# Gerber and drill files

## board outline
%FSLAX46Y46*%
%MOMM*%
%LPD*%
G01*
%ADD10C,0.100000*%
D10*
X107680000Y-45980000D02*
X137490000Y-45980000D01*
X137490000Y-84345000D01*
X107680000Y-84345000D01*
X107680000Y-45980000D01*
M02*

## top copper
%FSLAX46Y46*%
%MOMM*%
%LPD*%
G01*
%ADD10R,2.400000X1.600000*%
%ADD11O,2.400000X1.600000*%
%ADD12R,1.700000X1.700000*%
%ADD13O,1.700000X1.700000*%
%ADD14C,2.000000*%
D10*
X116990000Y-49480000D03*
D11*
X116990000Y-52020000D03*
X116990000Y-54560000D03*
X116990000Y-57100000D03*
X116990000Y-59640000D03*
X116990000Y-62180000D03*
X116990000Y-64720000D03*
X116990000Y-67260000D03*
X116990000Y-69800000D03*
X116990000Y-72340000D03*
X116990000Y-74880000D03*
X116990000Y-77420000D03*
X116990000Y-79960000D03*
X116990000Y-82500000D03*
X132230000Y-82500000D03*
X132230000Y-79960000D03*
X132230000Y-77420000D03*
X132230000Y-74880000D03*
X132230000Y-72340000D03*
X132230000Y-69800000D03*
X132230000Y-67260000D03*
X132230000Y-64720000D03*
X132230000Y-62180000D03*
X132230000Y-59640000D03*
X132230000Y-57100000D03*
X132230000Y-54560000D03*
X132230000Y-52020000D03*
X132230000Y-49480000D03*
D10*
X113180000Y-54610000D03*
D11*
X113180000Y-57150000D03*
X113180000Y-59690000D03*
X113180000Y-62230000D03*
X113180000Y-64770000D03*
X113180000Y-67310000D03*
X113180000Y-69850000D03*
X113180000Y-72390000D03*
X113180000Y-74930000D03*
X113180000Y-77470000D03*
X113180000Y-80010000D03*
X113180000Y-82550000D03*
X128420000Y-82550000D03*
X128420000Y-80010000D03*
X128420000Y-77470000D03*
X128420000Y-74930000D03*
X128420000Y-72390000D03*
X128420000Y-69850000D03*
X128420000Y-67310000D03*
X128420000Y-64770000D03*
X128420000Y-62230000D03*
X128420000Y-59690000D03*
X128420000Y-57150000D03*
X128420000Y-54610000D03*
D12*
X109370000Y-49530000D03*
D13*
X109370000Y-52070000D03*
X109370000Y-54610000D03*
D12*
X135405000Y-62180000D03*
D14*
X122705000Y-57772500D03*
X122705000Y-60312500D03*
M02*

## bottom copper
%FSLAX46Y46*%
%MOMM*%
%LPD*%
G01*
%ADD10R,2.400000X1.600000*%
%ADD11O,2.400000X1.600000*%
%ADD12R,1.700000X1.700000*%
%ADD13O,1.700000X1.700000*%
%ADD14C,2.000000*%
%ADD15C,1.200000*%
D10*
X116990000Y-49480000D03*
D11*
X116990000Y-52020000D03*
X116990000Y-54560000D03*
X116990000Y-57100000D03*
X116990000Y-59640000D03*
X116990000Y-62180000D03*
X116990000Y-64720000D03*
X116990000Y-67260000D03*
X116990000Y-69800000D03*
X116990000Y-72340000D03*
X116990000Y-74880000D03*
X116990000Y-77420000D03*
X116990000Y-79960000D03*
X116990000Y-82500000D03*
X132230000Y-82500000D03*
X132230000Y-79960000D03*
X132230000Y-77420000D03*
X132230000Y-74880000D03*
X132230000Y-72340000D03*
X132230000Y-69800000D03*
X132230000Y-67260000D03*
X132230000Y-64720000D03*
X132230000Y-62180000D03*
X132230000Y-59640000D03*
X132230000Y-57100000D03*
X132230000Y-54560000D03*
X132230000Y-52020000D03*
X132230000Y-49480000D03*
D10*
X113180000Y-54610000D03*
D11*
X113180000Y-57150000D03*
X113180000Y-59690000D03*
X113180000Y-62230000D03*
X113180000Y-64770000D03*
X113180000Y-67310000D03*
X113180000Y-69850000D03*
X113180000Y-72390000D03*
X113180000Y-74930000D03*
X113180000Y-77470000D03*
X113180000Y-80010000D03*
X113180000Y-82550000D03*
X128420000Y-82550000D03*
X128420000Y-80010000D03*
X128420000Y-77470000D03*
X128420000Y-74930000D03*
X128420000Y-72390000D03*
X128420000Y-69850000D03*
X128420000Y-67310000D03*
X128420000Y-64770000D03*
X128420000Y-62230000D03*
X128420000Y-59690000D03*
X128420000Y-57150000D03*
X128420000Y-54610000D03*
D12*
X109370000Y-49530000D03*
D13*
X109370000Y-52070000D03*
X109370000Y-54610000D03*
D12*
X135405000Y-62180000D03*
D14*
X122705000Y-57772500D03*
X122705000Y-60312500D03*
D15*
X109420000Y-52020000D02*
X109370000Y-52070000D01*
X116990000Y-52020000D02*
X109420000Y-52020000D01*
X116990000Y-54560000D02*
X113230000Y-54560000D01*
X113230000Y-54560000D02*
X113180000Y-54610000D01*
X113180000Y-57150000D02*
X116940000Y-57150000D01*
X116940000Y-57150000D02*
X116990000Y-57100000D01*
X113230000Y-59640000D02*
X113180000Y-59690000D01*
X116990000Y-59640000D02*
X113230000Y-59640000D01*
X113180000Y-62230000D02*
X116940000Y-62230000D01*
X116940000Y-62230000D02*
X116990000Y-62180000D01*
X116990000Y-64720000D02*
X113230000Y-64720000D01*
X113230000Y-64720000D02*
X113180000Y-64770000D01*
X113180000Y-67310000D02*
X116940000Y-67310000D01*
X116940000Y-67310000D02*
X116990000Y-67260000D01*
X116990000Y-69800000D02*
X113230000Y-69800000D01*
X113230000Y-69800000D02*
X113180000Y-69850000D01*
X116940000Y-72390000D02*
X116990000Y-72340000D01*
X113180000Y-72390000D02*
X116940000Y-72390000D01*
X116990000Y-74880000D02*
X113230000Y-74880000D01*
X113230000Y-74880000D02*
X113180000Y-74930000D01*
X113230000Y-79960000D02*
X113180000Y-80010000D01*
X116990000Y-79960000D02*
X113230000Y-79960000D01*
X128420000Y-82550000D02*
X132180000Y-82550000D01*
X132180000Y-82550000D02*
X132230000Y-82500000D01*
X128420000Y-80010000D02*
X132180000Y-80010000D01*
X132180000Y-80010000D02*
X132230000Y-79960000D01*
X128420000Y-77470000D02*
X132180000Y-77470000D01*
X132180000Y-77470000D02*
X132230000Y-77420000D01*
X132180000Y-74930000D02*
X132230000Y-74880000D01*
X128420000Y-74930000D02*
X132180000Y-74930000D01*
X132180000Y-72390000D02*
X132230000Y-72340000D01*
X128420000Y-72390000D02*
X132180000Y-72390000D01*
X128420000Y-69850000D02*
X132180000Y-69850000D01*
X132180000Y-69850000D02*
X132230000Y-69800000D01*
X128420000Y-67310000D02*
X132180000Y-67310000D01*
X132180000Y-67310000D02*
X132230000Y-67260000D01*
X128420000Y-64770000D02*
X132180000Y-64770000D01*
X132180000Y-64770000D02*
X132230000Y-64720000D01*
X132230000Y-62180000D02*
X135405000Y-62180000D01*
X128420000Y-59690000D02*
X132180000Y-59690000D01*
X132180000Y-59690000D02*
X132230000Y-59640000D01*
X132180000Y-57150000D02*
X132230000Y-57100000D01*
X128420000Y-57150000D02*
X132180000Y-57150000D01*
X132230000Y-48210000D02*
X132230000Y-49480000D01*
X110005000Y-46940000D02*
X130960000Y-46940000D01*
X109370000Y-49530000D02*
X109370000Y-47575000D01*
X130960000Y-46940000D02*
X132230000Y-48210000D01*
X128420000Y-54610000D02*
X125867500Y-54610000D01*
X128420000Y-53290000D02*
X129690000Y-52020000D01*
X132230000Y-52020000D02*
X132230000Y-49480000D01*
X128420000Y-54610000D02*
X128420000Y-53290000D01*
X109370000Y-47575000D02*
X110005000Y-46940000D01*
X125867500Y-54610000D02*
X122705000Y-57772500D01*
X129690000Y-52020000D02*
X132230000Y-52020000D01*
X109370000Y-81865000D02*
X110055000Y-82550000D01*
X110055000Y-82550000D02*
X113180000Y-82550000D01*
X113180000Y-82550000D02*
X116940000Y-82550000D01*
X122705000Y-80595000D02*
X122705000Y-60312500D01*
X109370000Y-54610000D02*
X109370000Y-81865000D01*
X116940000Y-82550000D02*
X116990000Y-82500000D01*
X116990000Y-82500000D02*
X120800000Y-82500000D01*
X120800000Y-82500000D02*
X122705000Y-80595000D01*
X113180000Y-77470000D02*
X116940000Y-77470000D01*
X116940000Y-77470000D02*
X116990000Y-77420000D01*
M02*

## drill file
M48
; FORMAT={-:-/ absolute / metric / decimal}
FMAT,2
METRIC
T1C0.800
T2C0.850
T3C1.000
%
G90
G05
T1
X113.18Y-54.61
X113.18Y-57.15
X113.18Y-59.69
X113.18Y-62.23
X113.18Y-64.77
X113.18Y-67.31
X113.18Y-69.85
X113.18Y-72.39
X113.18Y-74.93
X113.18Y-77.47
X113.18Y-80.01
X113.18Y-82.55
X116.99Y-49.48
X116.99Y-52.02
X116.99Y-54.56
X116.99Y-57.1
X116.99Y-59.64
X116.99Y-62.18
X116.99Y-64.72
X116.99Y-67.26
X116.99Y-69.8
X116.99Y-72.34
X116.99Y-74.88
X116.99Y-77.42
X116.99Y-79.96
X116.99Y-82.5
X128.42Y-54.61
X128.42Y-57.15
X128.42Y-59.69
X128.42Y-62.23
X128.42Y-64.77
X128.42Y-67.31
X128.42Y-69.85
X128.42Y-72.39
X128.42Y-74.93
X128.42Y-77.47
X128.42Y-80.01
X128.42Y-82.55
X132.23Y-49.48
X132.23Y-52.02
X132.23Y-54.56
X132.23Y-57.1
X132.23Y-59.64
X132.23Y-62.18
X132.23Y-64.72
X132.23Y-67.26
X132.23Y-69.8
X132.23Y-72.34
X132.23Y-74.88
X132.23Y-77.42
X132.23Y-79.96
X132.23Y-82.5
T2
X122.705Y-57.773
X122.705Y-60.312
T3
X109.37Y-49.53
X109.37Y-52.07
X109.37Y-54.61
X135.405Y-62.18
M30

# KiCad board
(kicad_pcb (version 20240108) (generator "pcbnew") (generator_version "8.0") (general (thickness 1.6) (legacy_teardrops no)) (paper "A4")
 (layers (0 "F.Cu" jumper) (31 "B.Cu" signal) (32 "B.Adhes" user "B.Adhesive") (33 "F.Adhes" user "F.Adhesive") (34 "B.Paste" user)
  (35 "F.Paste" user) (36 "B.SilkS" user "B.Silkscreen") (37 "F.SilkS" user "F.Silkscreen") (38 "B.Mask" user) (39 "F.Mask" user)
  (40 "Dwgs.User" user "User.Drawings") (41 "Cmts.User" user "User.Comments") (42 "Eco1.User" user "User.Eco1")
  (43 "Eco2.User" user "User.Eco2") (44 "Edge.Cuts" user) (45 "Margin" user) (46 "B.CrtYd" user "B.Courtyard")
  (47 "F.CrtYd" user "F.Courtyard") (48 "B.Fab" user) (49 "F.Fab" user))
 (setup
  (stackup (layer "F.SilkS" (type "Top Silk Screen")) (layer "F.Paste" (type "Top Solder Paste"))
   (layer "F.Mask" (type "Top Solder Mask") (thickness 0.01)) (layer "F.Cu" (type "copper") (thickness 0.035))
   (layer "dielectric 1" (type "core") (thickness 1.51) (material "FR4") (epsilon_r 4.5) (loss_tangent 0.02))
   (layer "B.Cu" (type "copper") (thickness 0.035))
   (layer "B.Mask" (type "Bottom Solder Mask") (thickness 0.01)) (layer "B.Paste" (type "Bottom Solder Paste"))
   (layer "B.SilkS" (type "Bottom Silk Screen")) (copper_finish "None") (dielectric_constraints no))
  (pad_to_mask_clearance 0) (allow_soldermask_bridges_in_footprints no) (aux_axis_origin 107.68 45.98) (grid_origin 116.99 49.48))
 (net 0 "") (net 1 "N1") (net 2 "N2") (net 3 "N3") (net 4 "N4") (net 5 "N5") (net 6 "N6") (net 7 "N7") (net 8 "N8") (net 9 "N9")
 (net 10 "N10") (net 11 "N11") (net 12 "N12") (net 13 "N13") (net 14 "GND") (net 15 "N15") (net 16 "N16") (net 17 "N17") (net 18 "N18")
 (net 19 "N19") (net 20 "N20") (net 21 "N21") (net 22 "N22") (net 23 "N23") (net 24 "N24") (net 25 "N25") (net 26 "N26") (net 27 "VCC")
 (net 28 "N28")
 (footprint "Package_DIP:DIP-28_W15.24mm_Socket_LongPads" (layer "F.Cu") (at 116.99 49.48)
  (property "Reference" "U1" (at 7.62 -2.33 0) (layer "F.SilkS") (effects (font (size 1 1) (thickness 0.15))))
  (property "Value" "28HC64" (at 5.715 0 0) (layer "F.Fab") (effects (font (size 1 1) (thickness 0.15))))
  (pad "1" thru_hole rect (at 0 0) (size 2.4 1.6) (drill 0.8) (layers "*.Cu" "*.Mask") (remove_unused_layers no) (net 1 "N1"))
  (pad "2" thru_hole oval (at 0 2.54) (size 2.4 1.6) (drill 0.8) (layers "*.Cu" "*.Mask") (remove_unused_layers no) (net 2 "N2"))
  (pad "3" thru_hole oval (at 0 5.08) (size 2.4 1.6) (drill 0.8) (layers "*.Cu" "*.Mask") (remove_unused_layers no) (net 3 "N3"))
  (pad "4" thru_hole oval (at 0 7.62) (size 2.4 1.6) (drill 0.8) (layers "*.Cu" "*.Mask") (remove_unused_layers no) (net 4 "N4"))
  (pad "5" thru_hole oval (at 0 10.16) (size 2.4 1.6) (drill 0.8) (layers "*.Cu" "*.Mask") (remove_unused_layers no) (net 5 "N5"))
  (pad "6" thru_hole oval (at 0 12.7) (size 2.4 1.6) (drill 0.8) (layers "*.Cu" "*.Mask") (remove_unused_layers no) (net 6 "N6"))
  (pad "7" thru_hole oval (at 0 15.24) (size 2.4 1.6) (drill 0.8) (layers "*.Cu" "*.Mask") (remove_unused_layers no) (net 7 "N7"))
  (pad "8" thru_hole oval (at 0 17.78) (size 2.4 1.6) (drill 0.8) (layers "*.Cu" "*.Mask") (remove_unused_layers no) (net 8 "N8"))
  (pad "9" thru_hole oval (at 0 20.32) (size 2.4 1.6) (drill 0.8) (layers "*.Cu" "*.Mask") (remove_unused_layers no) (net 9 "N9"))
  (pad "10" thru_hole oval (at 0 22.86) (size 2.4 1.6) (drill 0.8) (layers "*.Cu" "*.Mask") (remove_unused_layers no) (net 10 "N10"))
  (pad "11" thru_hole oval (at 0 25.4) (size 2.4 1.6) (drill 0.8) (layers "*.Cu" "*.Mask") (remove_unused_layers no) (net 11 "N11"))
  (pad "12" thru_hole oval (at 0 27.94) (size 2.4 1.6) (drill 0.8) (layers "*.Cu" "*.Mask") (remove_unused_layers no) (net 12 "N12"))
  (pad "13" thru_hole oval (at 0 30.48) (size 2.4 1.6) (drill 0.8) (layers "*.Cu" "*.Mask") (remove_unused_layers no) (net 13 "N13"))
  (pad "14" thru_hole oval (at 0 33.02) (size 2.4 1.6) (drill 0.8) (layers "*.Cu" "*.Mask") (remove_unused_layers no) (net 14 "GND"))
  (pad "15" thru_hole oval (at 15.24 33.02) (size 2.4 1.6) (drill 0.8) (layers "*.Cu" "*.Mask") (remove_unused_layers no) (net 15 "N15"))
  (pad "16" thru_hole oval (at 15.24 30.48) (size 2.4 1.6) (drill 0.8) (layers "*.Cu" "*.Mask") (remove_unused_layers no) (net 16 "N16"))
  (pad "17" thru_hole oval (at 15.24 27.94) (size 2.4 1.6) (drill 0.8) (layers "*.Cu" "*.Mask") (remove_unused_layers no) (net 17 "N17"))
  (pad "18" thru_hole oval (at 15.24 25.4) (size 2.4 1.6) (drill 0.8) (layers "*.Cu" "*.Mask") (remove_unused_layers no) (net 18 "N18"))
  (pad "19" thru_hole oval (at 15.24 22.86) (size 2.4 1.6) (drill 0.8) (layers "*.Cu" "*.Mask") (remove_unused_layers no) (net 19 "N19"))
  (pad "20" thru_hole oval (at 15.24 20.32) (size 2.4 1.6) (drill 0.8) (layers "*.Cu" "*.Mask") (remove_unused_layers no) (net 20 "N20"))
  (pad "21" thru_hole oval (at 15.24 17.78) (size 2.4 1.6) (drill 0.8) (layers "*.Cu" "*.Mask") (remove_unused_layers no) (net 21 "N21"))
  (pad "22" thru_hole oval (at 15.24 15.24) (size 2.4 1.6) (drill 0.8) (layers "*.Cu" "*.Mask") (remove_unused_layers no) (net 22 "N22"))
  (pad "23" thru_hole oval (at 15.24 12.7) (size 2.4 1.6) (drill 0.8) (layers "*.Cu" "*.Mask") (remove_unused_layers no) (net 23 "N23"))
  (pad "24" thru_hole oval (at 15.24 10.16) (size 2.4 1.6) (drill 0.8) (layers "*.Cu" "*.Mask") (remove_unused_layers no) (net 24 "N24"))
  (pad "25" thru_hole oval (at 15.24 7.62) (size 2.4 1.6) (drill 0.8) (layers "*.Cu" "*.Mask") (remove_unused_layers no) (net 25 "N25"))
  (pad "26" thru_hole oval (at 15.24 5.08) (size 2.4 1.6) (drill 0.8) (layers "*.Cu" "*.Mask") (remove_unused_layers no) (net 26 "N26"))
  (pad "27" thru_hole oval (at 15.24 2.54) (size 2.4 1.6) (drill 0.8) (layers "*.Cu" "*.Mask") (remove_unused_layers no) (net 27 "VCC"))
  (pad "28" thru_hole oval (at 15.24 0) (size 2.4 1.6) (drill 0.8) (layers "*.Cu" "*.Mask") (remove_unused_layers no) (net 27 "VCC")))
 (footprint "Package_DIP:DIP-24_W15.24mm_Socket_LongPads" (layer "F.Cu") (at 113.18 54.61)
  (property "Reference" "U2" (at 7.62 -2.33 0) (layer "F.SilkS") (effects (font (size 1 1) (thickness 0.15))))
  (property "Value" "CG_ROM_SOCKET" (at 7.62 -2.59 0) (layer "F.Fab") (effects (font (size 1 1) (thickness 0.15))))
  (pad "1" thru_hole rect (at 0 0) (size 2.4 1.6) (drill 0.8) (layers "*.Cu" "*.Mask") (remove_unused_layers no) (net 3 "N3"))
  (pad "2" thru_hole oval (at 0 2.54) (size 2.4 1.6) (drill 0.8) (layers "*.Cu" "*.Mask") (remove_unused_layers no) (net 4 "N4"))
  (pad "3" thru_hole oval (at 0 5.08) (size 2.4 1.6) (drill 0.8) (layers "*.Cu" "*.Mask") (remove_unused_layers no) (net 5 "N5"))
  (pad "4" thru_hole oval (at 0 7.62) (size 2.4 1.6) (drill 0.8) (layers "*.Cu" "*.Mask") (remove_unused_layers no) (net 6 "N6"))
  (pad "5" thru_hole oval (at 0 10.16) (size 2.4 1.6) (drill 0.8) (layers "*.Cu" "*.Mask") (remove_unused_layers no) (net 7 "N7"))
  (pad "6" thru_hole oval (at 0 12.7) (size 2.4 1.6) (drill 0.8) (layers "*.Cu" "*.Mask") (remove_unused_layers no) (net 8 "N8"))
  (pad "7" thru_hole oval (at 0 15.24) (size 2.4 1.6) (drill 0.8) (layers "*.Cu" "*.Mask") (remove_unused_layers no) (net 9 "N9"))
  (pad "8" thru_hole oval (at 0 17.78) (size 2.4 1.6) (drill 0.8) (layers "*.Cu" "*.Mask") (remove_unused_layers no) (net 10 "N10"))
  (pad "9" thru_hole oval (at 0 20.32) (size 2.4 1.6) (drill 0.8) (layers "*.Cu" "*.Mask") (remove_unused_layers no) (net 11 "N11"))
  (pad "10" thru_hole oval (at 0 22.86) (size 2.4 1.6) (drill 0.8) (layers "*.Cu" "*.Mask") (remove_unused_layers no) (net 12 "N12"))
  (pad "11" thru_hole oval (at 0 25.4) (size 2.4 1.6) (drill 0.8) (layers "*.Cu" "*.Mask") (remove_unused_layers no) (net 13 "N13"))
  (pad "12" thru_hole oval (at 0 27.94) (size 2.4 1.6) (drill 0.8) (layers "*.Cu" "*.Mask") (remove_unused_layers no) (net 14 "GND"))
  (pad "13" thru_hole oval (at 15.24 27.94) (size 2.4 1.6) (drill 0.8) (layers "*.Cu" "*.Mask") (remove_unused_layers no) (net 15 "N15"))
  (pad "14" thru_hole oval (at 15.24 25.4) (size 2.4 1.6) (drill 0.8) (layers "*.Cu" "*.Mask") (remove_unused_layers no) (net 16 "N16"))
  (pad "15" thru_hole oval (at 15.24 22.86) (size 2.4 1.6) (drill 0.8) (layers "*.Cu" "*.Mask") (remove_unused_layers no) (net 17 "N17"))
  (pad "16" thru_hole oval (at 15.24 20.32) (size 2.4 1.6) (drill 0.8) (layers "*.Cu" "*.Mask") (remove_unused_layers no) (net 18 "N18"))
  (pad "17" thru_hole oval (at 15.24 17.78) (size 2.4 1.6) (drill 0.8) (layers "*.Cu" "*.Mask") (remove_unused_layers no) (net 19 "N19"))
  (pad "18" thru_hole oval (at 15.24 15.24) (size 2.4 1.6) (drill 0.8) (layers "*.Cu" "*.Mask") (remove_unused_layers no) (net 20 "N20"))
  (pad "19" thru_hole oval (at 15.24 12.7) (size 2.4 1.6) (drill 0.8) (layers "*.Cu" "*.Mask") (remove_unused_layers no) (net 21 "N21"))
  (pad "20" thru_hole oval (at 15.24 10.16) (size 2.4 1.6) (drill 0.8) (layers "*.Cu" "*.Mask") (remove_unused_layers no) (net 22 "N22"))
  (pad "21" thru_hole oval (at 15.24 7.62) (size 2.4 1.6) (drill 0.8) (layers "*.Cu" "*.Mask") (remove_unused_layers no) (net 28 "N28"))
  (pad "22" thru_hole oval (at 15.24 5.08) (size 2.4 1.6) (drill 0.8) (layers "*.Cu" "*.Mask") (remove_unused_layers no) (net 24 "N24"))
  (pad "23" thru_hole oval (at 15.24 2.54) (size 2.4 1.6) (drill 0.8) (layers "*.Cu" "*.Mask") (remove_unused_layers no) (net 25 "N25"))
  (pad "24" thru_hole oval (at 15.24 0) (size 2.4 1.6) (drill 0.8) (layers "*.Cu" "*.Mask") (remove_unused_layers no) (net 27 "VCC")))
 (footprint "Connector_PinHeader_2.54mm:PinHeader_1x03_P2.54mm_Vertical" (layer "F.Cu") (at 109.37 49.53)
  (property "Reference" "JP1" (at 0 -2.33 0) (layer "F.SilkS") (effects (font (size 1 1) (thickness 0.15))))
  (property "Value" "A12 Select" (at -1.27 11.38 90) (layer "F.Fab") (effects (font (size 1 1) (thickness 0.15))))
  (pad "1" thru_hole rect (at 0 0) (size 1.7 1.7) (drill 1) (layers "*.Cu" "*.Mask") (remove_unused_layers no) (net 27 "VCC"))
  (pad "2" thru_hole oval (at 0 2.54) (size 1.7 1.7) (drill 1) (layers "*.Cu" "*.Mask") (remove_unused_layers no) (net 2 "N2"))
  (pad "3" thru_hole oval (at 0 5.08) (size 1.7 1.7) (drill 1) (layers "*.Cu" "*.Mask") (remove_unused_layers no) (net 14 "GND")))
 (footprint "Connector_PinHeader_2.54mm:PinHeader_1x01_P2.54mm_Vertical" (layer "F.Cu") (at 135.405 62.18)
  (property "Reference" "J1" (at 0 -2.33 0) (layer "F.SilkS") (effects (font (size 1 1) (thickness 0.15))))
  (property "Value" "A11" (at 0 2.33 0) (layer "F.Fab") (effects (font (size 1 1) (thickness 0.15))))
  (pad "1" thru_hole rect (at 0 0) (size 1.7 1.7) (drill 1) (layers "*.Cu" "*.Mask") (remove_unused_layers no) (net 23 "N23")))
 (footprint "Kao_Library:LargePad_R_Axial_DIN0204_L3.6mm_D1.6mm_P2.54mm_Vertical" (layer "F.Cu") (at 122.705 57.7725 -90)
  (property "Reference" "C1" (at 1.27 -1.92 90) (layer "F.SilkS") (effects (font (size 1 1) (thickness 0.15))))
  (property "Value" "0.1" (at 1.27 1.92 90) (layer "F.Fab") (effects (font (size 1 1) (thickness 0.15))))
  (pad "1" thru_hole circle (at 0 0 270) (size 2 2) (drill 0.85) (layers "*.Cu" "*.Mask") (remove_unused_layers no) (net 27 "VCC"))
  (pad "2" thru_hole circle (at 2.54 0 270) (size 2 2) (drill 0.85) (layers "*.Cu" "*.Mask") (remove_unused_layers no) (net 14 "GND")))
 (gr_rect (start 107.68 45.98) (end 137.49 84.345) (stroke (width 0.1) (type default)) (fill none) (layer "Edge.Cuts"))
 (segment (start 109.42 52.02) (end 109.37 52.07) (width 1.2) (layer "B.Cu") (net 2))
 (segment (start 116.99 52.02) (end 109.42 52.02) (width 1.2) (layer "B.Cu") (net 2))
 (segment (start 116.99 54.56) (end 113.23 54.56) (width 1.2) (layer "B.Cu") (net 3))
 (segment (start 113.23 54.56) (end 113.18 54.61) (width 1.2) (layer "B.Cu") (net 3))
 (segment (start 113.18 57.15) (end 116.94 57.15) (width 1.2) (layer "B.Cu") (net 4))
 (segment (start 116.94 57.15) (end 116.99 57.1) (width 1.2) (layer "B.Cu") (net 4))
 (segment (start 113.23 59.64) (end 113.18 59.69) (width 1.2) (layer "B.Cu") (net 5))
 (segment (start 116.99 59.64) (end 113.23 59.64) (width 1.2) (layer "B.Cu") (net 5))
 (segment (start 113.18 62.23) (end 116.94 62.23) (width 1.2) (layer "B.Cu") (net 6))
 (segment (start 116.94 62.23) (end 116.99 62.18) (width 1.2) (layer "B.Cu") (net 6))
 (segment (start 116.99 64.72) (end 113.23 64.72) (width 1.2) (layer "B.Cu") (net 7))
 (segment (start 113.23 64.72) (end 113.18 64.77) (width 1.2) (layer "B.Cu") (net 7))
 (segment (start 113.18 67.31) (end 116.94 67.31) (width 1.2) (layer "B.Cu") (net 8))
 (segment (start 116.94 67.31) (end 116.99 67.26) (width 1.2) (layer "B.Cu") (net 8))
 (segment (start 116.99 69.8) (end 113.23 69.8) (width 1.2) (layer "B.Cu") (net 9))
 (segment (start 113.23 69.8) (end 113.18 69.85) (width 1.2) (layer "B.Cu") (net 9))
 (segment (start 116.94 72.39) (end 116.99 72.34) (width 1.2) (layer "B.Cu") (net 10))
 (segment (start 113.18 72.39) (end 116.94 72.39) (width 1.2) (layer "B.Cu") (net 10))
 (segment (start 116.99 74.88) (end 113.23 74.88) (width 1.2) (layer "B.Cu") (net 11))
 (segment (start 113.23 74.88) (end 113.18 74.93) (width 1.2) (layer "B.Cu") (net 11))
 (segment (start 113.23 79.96) (end 113.18 80.01) (width 1.2) (layer "B.Cu") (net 13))
 (segment (start 116.99 79.96) (end 113.23 79.96) (width 1.2) (layer "B.Cu") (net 13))
 (segment (start 128.42 82.55) (end 132.18 82.55) (width 1.2) (layer "B.Cu") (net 15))
 (segment (start 132.18 82.55) (end 132.23 82.5) (width 1.2) (layer "B.Cu") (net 15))
 (segment (start 128.42 80.01) (end 132.18 80.01) (width 1.2) (layer "B.Cu") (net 16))
 (segment (start 132.18 80.01) (end 132.23 79.96) (width 1.2) (layer "B.Cu") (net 16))
 (segment (start 128.42 77.47) (end 132.18 77.47) (width 1.2) (layer "B.Cu") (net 17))
 (segment (start 132.18 77.47) (end 132.23 77.42) (width 1.2) (layer "B.Cu") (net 17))
 (segment (start 132.18 74.93) (end 132.23 74.88) (width 1.2) (layer "B.Cu") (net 18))
 (segment (start 128.42 74.93) (end 132.18 74.93) (width 1.2) (layer "B.Cu") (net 18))
 (segment (start 132.18 72.39) (end 132.23 72.34) (width 1.2) (layer "B.Cu") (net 19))
 (segment (start 128.42 72.39) (end 132.18 72.39) (width 1.2) (layer "B.Cu") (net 19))
 (segment (start 128.42 69.85) (end 132.18 69.85) (width 1.2) (layer "B.Cu") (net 20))
 (segment (start 132.18 69.85) (end 132.23 69.8) (width 1.2) (layer "B.Cu") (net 20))
 (segment (start 128.42 67.31) (end 132.18 67.31) (width 1.2) (layer "B.Cu") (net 21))
 (segment (start 132.18 67.31) (end 132.23 67.26) (width 1.2) (layer "B.Cu") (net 21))
 (segment (start 128.42 64.77) (end 132.18 64.77) (width 1.2) (layer "B.Cu") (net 22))
 (segment (start 132.18 64.77) (end 132.23 64.72) (width 1.2) (layer "B.Cu") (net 22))
 (segment (start 132.23 62.18) (end 135.405 62.18) (width 1.2) (layer "B.Cu") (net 23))
 (segment (start 128.42 59.69) (end 132.18 59.69) (width 1.2) (layer "B.Cu") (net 24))
 (segment (start 132.18 59.69) (end 132.23 59.64) (width 1.2) (layer "B.Cu") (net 24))
 (segment (start 132.18 57.15) (end 132.23 57.1) (width 1.2) (layer "B.Cu") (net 25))
 (segment (start 128.42 57.15) (end 132.18 57.15) (width 1.2) (layer "B.Cu") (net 25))
 (segment (start 132.23 48.21) (end 132.23 49.48) (width 1.2) (layer "B.Cu") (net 27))
 (segment (start 110.005 46.94) (end 130.96 46.94) (width 1.2) (layer "B.Cu") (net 27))
 (segment (start 109.37 49.53) (end 109.37 47.575) (width 1.2) (layer "B.Cu") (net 27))
 (segment (start 130.96 46.94) (end 132.23 48.21) (width 1.2) (layer "B.Cu") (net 27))
 (segment (start 128.42 54.61) (end 125.8675 54.61) (width 1.2) (layer "B.Cu") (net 27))
 (segment (start 128.42 53.29) (end 129.69 52.02) (width 1.2) (layer "B.Cu") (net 27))
 (segment (start 132.23 52.02) (end 132.23 49.48) (width 1.2) (layer "B.Cu") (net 27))
 (segment (start 128.42 54.61) (end 128.42 53.29) (width 1.2) (layer "B.Cu") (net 27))
 (segment (start 109.37 47.575) (end 110.005 46.94) (width 1.2) (layer "B.Cu") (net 27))
 (segment (start 125.8675 54.61) (end 122.705 57.7725) (width 1.2) (layer "B.Cu") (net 27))
 (segment (start 129.69 52.02) (end 132.23 52.02) (width 1.2) (layer "B.Cu") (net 27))
 (segment (start 109.37 81.865) (end 110.055 82.55) (width 1.2) (layer "B.Cu") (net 14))
 (segment (start 110.055 82.55) (end 113.18 82.55) (width 1.2) (layer "B.Cu") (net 14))
 (segment (start 113.18 82.55) (end 116.94 82.55) (width 1.2) (layer "B.Cu") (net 14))
 (segment (start 122.705 80.595) (end 122.705 60.3125) (width 1.2) (layer "B.Cu") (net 14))
 (segment (start 109.37 54.61) (end 109.37 81.865) (width 1.2) (layer "B.Cu") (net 14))
 (segment (start 116.94 82.55) (end 116.99 82.5) (width 1.2) (layer "B.Cu") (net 14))
 (segment (start 116.99 82.5) (end 120.8 82.5) (width 1.2) (layer "B.Cu") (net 14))
 (segment (start 120.8 82.5) (end 122.705 80.595) (width 1.2) (layer "B.Cu") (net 14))
 (segment (start 113.18 77.47) (end 116.94 77.47) (width 1.2) (layer "B.Cu") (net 12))
 (segment (start 116.94 77.47) (end 116.99 77.42) (width 1.2) (layer "B.Cu") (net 12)))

